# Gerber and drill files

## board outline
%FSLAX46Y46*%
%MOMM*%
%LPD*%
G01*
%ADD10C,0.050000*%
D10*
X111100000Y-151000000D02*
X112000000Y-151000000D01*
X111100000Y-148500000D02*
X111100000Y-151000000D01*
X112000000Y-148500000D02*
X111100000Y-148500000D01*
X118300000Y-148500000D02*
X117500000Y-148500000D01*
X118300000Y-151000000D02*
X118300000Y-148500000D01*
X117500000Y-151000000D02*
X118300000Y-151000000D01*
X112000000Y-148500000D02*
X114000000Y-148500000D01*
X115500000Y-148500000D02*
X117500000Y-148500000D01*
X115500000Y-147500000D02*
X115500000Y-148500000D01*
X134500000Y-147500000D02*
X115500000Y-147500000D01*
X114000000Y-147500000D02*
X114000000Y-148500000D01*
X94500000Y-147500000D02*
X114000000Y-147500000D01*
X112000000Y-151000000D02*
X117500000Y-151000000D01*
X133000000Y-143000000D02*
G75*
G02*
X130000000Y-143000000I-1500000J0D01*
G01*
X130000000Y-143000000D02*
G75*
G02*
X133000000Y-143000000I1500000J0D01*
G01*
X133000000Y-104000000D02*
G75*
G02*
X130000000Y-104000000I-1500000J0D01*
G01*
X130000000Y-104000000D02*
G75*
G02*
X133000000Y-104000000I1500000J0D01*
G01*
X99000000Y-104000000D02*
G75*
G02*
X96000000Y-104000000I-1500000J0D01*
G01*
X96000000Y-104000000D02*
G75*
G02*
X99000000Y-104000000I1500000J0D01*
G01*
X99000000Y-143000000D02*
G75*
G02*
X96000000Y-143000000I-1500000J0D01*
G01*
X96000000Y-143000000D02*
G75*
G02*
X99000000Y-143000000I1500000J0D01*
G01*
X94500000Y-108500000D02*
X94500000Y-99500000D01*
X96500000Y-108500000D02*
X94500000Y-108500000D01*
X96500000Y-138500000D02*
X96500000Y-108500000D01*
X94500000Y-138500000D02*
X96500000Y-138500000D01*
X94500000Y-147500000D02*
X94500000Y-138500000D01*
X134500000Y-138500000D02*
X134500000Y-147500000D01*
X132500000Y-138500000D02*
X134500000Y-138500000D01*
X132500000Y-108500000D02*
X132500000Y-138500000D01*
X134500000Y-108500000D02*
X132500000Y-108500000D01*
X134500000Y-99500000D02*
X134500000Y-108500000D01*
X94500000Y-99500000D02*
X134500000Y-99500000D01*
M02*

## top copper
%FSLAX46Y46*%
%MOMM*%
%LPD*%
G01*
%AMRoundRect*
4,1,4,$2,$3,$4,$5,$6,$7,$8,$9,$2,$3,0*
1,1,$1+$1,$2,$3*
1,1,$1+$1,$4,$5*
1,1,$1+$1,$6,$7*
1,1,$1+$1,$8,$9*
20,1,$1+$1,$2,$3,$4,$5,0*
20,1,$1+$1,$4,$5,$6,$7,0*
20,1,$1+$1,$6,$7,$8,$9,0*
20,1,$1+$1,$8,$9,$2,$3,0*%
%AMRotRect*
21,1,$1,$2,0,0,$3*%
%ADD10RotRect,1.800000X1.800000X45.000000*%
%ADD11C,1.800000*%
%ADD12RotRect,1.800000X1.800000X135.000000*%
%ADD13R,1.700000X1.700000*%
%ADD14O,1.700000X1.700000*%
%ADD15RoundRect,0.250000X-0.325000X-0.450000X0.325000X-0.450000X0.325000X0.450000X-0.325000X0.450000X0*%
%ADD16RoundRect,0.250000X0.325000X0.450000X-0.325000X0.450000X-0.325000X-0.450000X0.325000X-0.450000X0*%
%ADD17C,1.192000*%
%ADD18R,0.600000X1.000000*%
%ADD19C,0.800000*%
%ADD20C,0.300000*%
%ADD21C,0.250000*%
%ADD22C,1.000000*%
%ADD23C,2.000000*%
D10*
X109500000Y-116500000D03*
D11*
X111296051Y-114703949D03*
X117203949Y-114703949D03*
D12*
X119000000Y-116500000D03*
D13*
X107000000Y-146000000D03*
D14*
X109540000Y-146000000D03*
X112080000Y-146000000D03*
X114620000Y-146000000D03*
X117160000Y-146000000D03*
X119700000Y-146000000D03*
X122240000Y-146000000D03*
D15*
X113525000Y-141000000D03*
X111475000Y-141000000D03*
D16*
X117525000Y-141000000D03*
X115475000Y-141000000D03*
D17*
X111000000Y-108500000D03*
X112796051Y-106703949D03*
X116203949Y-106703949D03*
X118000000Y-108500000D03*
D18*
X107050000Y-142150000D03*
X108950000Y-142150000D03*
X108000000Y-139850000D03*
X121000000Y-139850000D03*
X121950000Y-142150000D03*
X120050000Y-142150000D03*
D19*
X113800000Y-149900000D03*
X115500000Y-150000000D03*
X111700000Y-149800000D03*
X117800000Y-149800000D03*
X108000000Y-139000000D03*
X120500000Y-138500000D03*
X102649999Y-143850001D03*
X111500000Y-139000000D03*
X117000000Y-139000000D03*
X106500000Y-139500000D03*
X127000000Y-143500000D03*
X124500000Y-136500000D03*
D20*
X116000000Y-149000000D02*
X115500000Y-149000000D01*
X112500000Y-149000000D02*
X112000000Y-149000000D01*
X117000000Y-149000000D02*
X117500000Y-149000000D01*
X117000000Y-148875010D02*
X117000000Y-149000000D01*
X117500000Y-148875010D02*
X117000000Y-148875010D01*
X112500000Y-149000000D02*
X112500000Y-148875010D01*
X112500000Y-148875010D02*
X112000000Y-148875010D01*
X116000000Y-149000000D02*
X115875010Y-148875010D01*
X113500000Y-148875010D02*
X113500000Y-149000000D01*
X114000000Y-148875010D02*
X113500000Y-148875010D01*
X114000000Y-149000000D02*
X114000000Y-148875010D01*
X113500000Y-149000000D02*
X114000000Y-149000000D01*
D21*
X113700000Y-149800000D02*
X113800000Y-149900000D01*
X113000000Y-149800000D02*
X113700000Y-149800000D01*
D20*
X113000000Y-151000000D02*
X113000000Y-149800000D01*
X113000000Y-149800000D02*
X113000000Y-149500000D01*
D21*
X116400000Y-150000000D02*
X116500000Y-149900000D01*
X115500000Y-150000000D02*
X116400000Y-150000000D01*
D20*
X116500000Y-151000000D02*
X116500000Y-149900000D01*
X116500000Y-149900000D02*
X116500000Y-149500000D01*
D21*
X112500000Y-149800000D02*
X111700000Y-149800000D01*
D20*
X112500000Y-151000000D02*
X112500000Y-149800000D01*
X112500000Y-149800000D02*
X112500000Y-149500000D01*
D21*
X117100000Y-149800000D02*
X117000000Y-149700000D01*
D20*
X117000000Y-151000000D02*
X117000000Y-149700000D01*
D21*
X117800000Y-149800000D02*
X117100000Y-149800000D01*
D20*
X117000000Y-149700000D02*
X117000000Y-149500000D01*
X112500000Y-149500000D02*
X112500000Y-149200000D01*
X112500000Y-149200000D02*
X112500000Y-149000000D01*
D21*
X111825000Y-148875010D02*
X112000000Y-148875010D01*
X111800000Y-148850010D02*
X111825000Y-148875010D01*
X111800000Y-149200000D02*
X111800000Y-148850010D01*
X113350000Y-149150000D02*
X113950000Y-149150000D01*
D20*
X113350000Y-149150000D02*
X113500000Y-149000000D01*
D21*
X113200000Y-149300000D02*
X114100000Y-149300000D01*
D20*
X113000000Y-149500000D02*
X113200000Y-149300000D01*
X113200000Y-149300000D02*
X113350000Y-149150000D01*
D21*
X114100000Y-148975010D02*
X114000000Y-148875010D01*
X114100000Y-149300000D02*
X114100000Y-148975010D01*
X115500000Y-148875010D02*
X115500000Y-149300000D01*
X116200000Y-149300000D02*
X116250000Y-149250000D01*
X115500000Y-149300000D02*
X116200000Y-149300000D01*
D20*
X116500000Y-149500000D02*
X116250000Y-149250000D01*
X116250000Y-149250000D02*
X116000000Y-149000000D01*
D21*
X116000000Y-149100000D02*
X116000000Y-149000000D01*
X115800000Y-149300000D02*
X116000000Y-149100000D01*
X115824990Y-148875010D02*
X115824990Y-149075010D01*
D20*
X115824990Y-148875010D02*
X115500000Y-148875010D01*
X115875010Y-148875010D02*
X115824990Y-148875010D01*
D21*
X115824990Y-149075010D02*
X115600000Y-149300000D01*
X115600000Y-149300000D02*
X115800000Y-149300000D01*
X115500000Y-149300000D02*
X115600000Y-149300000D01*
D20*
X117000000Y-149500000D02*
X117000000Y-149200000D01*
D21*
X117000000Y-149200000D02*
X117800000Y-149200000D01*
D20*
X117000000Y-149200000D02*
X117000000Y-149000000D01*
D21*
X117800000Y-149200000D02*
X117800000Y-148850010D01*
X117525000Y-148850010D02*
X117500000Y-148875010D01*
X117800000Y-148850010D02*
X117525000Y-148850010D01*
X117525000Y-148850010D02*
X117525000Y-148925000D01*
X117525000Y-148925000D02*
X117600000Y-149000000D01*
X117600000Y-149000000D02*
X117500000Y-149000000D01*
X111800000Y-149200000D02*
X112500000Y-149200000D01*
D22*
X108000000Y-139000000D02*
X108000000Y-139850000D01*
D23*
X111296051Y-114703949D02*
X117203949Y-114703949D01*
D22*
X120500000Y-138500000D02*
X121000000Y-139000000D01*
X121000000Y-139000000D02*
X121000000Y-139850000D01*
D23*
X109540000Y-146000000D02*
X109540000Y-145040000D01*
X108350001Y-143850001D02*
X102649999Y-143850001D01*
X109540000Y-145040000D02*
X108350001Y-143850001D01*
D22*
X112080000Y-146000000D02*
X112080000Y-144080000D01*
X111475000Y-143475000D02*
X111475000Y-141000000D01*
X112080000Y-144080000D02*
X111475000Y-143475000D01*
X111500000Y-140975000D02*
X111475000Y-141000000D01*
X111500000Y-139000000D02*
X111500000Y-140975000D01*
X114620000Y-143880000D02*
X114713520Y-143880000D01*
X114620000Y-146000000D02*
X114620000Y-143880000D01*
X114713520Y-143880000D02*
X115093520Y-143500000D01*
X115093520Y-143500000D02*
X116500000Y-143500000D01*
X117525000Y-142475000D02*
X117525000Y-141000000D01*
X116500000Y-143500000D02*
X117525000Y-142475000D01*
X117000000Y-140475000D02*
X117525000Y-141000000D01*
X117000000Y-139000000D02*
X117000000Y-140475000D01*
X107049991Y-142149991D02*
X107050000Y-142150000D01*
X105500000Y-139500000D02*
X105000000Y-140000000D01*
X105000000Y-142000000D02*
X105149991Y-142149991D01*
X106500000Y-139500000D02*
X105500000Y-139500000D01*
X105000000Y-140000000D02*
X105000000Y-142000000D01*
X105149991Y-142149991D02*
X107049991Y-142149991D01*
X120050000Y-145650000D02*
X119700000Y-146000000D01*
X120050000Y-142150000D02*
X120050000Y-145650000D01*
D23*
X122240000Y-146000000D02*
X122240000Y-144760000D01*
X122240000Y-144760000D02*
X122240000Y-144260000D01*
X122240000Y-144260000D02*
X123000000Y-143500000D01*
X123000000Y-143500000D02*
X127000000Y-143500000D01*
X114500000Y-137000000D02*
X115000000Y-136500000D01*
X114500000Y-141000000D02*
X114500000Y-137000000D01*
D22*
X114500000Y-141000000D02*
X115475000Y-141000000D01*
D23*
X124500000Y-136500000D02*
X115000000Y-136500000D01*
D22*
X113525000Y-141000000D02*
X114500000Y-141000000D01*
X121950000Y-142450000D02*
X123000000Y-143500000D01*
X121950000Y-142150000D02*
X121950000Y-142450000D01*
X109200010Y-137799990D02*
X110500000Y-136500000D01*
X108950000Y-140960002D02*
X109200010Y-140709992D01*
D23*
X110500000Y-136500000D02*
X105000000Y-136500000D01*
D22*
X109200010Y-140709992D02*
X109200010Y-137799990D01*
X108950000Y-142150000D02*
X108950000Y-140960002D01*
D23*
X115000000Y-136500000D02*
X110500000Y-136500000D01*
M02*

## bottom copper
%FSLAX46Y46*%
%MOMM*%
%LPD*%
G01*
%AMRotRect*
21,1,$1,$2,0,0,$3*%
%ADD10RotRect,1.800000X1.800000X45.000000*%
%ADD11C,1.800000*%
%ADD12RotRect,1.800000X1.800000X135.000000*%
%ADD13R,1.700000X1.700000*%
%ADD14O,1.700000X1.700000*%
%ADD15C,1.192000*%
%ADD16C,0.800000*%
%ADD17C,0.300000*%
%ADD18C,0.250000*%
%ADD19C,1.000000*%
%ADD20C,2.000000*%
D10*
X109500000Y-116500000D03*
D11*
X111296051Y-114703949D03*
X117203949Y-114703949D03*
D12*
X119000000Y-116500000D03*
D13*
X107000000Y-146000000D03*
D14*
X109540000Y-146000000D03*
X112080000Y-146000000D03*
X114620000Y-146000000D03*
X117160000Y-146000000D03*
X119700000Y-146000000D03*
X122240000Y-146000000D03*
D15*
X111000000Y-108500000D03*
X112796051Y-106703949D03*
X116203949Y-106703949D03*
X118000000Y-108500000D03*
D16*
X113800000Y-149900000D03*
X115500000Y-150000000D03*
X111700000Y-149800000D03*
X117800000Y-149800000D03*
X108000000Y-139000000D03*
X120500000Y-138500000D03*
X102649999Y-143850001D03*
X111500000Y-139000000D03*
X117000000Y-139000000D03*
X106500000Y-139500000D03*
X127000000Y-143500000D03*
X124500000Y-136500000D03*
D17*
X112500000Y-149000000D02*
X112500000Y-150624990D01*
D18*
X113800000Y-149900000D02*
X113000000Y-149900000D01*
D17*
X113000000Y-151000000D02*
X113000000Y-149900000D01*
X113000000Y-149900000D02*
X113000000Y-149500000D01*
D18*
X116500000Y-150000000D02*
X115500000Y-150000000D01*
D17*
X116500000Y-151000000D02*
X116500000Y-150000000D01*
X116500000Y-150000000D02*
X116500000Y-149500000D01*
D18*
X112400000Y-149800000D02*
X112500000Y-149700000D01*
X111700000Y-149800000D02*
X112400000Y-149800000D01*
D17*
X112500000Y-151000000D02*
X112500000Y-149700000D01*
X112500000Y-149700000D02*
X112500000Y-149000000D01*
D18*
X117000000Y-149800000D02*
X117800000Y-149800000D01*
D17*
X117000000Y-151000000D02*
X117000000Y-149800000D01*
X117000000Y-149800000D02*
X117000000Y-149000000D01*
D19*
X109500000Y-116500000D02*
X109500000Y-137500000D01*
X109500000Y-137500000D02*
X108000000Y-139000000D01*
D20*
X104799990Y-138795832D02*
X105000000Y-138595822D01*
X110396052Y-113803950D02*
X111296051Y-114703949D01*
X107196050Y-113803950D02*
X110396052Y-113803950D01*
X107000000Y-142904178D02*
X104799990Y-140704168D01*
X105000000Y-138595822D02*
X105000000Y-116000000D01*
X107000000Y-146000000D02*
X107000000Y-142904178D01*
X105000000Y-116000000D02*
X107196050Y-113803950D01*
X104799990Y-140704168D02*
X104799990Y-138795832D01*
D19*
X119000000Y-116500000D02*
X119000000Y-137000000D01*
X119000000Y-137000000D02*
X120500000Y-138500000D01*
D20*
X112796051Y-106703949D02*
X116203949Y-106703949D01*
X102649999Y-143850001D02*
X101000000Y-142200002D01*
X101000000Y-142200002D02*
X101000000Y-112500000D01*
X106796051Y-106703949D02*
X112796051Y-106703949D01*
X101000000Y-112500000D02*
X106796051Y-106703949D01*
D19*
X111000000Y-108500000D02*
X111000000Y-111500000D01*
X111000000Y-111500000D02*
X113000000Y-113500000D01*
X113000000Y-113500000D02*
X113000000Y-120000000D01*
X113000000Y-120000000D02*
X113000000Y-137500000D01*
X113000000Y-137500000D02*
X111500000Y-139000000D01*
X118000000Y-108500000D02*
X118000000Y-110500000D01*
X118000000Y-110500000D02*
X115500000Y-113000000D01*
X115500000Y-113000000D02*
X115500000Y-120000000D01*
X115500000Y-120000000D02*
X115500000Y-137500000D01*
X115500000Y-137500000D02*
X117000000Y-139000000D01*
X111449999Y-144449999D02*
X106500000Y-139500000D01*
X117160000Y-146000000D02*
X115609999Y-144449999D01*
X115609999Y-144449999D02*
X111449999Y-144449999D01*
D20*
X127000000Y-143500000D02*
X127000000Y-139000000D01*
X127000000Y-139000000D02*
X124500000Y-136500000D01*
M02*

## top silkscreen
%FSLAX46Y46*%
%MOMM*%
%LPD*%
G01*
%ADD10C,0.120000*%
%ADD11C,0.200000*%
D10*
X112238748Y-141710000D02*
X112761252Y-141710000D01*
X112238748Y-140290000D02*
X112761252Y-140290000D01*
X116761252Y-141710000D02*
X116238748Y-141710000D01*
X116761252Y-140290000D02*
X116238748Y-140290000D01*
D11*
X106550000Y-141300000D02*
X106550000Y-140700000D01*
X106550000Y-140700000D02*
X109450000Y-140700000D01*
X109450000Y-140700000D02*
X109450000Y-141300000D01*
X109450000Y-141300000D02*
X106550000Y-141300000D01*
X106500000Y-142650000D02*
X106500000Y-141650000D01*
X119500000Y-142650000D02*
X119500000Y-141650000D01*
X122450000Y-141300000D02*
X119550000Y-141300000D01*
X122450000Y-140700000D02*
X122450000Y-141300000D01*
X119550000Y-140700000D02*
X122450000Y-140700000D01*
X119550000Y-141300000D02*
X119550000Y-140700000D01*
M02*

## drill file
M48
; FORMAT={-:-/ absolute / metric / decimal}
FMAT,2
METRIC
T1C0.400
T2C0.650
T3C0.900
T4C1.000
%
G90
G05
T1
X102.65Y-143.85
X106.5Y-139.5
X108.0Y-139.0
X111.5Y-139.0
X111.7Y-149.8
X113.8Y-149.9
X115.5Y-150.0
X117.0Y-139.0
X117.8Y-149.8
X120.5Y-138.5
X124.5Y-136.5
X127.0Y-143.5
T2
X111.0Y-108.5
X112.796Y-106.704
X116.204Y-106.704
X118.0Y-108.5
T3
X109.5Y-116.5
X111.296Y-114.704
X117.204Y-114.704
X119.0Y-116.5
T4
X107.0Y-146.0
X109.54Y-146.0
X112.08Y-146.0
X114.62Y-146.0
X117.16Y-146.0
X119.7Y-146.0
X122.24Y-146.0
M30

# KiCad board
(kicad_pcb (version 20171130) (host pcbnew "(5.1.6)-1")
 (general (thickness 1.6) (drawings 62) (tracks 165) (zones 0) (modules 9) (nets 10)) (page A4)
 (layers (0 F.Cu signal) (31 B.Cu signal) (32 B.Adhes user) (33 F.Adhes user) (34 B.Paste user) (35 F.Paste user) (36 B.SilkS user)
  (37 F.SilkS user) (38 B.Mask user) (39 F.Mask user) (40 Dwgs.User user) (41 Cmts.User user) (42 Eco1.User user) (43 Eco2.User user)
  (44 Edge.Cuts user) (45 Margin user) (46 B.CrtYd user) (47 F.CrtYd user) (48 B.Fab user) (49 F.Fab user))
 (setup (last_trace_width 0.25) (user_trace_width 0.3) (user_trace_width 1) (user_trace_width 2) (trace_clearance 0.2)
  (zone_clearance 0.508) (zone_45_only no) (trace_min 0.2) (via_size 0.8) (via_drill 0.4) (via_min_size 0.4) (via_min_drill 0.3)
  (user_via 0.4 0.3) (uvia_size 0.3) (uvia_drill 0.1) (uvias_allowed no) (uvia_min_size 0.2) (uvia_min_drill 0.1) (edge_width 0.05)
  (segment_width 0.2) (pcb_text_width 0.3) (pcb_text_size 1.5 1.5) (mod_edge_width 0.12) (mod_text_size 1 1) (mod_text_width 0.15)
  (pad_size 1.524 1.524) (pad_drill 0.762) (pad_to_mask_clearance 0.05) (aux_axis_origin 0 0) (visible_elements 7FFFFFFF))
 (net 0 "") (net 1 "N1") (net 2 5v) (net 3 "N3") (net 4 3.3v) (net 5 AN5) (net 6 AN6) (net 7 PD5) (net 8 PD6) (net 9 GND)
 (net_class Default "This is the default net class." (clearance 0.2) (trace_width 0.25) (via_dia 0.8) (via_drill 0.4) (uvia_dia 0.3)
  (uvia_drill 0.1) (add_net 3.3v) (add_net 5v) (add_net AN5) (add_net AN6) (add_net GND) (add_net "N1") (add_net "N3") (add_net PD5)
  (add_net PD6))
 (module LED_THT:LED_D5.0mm (layer B.Cu) (at 109.5 116.5 45)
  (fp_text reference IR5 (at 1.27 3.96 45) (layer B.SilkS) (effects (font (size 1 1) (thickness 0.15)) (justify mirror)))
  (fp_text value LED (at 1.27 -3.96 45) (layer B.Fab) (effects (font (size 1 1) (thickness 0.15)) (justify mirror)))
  (pad 1 thru_hole rect (at 0 0 45) (size 1.8 1.8) (drill 0.9) (layers *.Cu *.Mask) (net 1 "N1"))
  (pad 2 thru_hole circle (at 2.54 0 45) (size 1.8 1.8) (drill 0.9) (layers *.Cu *.Mask) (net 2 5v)))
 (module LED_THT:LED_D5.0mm (layer B.Cu) (at 119 116.5 135)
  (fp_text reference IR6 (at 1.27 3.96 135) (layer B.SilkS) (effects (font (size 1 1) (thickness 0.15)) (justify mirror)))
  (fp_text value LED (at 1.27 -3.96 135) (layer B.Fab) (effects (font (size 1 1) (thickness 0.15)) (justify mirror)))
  (pad 2 thru_hole circle (at 2.54 0 135) (size 1.8 1.8) (drill 0.9) (layers *.Cu *.Mask) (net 2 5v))
  (pad 1 thru_hole rect (at 0 0 135) (size 1.8 1.8) (drill 0.9) (layers *.Cu *.Mask) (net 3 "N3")))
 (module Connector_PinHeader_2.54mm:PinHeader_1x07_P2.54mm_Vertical (layer B.Cu) (at 107 146 270)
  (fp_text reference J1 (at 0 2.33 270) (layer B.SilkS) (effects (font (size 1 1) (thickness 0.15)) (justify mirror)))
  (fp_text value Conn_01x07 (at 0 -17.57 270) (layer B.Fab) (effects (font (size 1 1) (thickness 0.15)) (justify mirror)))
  (pad 1 thru_hole rect (at 0 0 270) (size 1.7 1.7) (drill 1) (layers *.Cu *.Mask) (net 2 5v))
  (pad 2 thru_hole oval (at 0 -2.54 270) (size 1.7 1.7) (drill 1) (layers *.Cu *.Mask) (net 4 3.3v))
  (pad 3 thru_hole oval (at 0 -5.08 270) (size 1.7 1.7) (drill 1) (layers *.Cu *.Mask) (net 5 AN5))
  (pad 4 thru_hole oval (at 0 -7.62 270) (size 1.7 1.7) (drill 1) (layers *.Cu *.Mask) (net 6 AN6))
  (pad 5 thru_hole oval (at 0 -10.16 270) (size 1.7 1.7) (drill 1) (layers *.Cu *.Mask) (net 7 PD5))
  (pad 6 thru_hole oval (at 0 -12.7 270) (size 1.7 1.7) (drill 1) (layers *.Cu *.Mask) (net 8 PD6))
  (pad 7 thru_hole oval (at 0 -15.24 270) (size 1.7 1.7) (drill 1) (layers *.Cu *.Mask) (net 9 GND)))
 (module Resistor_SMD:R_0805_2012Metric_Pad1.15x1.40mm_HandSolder (layer F.Cu) (at 112.5 141)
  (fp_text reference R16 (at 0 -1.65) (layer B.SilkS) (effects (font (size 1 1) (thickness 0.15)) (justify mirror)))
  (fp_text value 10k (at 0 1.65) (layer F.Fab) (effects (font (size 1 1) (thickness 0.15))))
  (fp_line (start -0.261252 0.71) (end 0.261252 0.71) (layer F.SilkS) (width 0.12))
  (fp_line (start -0.261252 -0.71) (end 0.261252 -0.71) (layer F.SilkS) (width 0.12))
  (pad 2 smd roundrect (at 1.025 0) (size 1.15 1.4) (layers F.Cu F.Paste F.Mask) (roundrect_rratio 0.217391) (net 9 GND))
  (pad 1 smd roundrect (at -1.025 0) (size 1.15 1.4) (layers F.Cu F.Paste F.Mask) (roundrect_rratio 0.217391) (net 5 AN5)))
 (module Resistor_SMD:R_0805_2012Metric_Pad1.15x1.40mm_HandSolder (layer F.Cu) (at 116.5 141 180)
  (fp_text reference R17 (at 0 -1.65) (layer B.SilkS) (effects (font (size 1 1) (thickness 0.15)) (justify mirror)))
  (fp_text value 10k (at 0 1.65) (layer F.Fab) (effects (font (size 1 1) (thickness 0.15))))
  (fp_line (start -0.261252 -0.71) (end 0.261252 -0.71) (layer F.SilkS) (width 0.12))
  (fp_line (start -0.261252 0.71) (end 0.261252 0.71) (layer F.SilkS) (width 0.12))
  (pad 1 smd roundrect (at -1.025 0 180) (size 1.15 1.4) (layers F.Cu F.Paste F.Mask) (roundrect_rratio 0.217391) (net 6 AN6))
  (pad 2 smd roundrect (at 1.025 0 180) (size 1.15 1.4) (layers F.Cu F.Paste F.Mask) (roundrect_rratio 0.217391) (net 9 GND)))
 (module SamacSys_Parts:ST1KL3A (layer B.Cu) (at 111 108.5 45)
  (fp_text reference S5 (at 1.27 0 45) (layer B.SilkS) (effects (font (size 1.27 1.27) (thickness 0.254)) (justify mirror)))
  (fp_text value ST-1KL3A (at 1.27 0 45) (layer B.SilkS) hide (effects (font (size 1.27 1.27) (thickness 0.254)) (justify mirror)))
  (pad 1 thru_hole circle (at 0 0 45) (size 1.192 1.192) (drill 0.65) (layers *.Cu *.Mask) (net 5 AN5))
  (pad 2 thru_hole circle (at 2.54 0 45) (size 1.192 1.192) (drill 0.65) (layers *.Cu *.Mask) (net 4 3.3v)))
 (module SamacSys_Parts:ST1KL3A (layer B.Cu) (at 118 108.5 135)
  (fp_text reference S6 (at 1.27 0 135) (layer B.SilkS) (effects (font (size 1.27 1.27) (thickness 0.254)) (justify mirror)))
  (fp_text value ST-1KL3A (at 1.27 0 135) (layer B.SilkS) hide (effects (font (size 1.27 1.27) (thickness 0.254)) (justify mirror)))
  (pad 2 thru_hole circle (at 2.54 0 135) (size 1.192 1.192) (drill 0.65) (layers *.Cu *.Mask) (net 4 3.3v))
  (pad 1 thru_hole circle (at 0 0 135) (size 1.192 1.192) (drill 0.65) (layers *.Cu *.Mask) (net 6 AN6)))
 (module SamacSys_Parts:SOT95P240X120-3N (layer F.Cu) (at 108 141 90)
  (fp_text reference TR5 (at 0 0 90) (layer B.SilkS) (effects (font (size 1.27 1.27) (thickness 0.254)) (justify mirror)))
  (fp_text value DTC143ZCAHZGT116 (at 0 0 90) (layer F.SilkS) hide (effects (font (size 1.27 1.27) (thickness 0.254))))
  (fp_line (start -0.3 -1.45) (end 0.3 -1.45) (layer F.SilkS) (width 0.2))
  (fp_line (start 0.3 -1.45) (end 0.3 1.45) (layer F.SilkS) (width 0.2))
  (fp_line (start 0.3 1.45) (end -0.3 1.45) (layer F.SilkS) (width 0.2))
  (fp_line (start -0.3 1.45) (end -0.3 -1.45) (layer F.SilkS) (width 0.2))
  (fp_line (start -1.65 -1.5) (end -0.65 -1.5) (layer F.SilkS) (width 0.2))
  (pad 1 smd rect (at -1.15 -0.95 180) (size 0.6 1) (layers F.Cu F.Paste F.Mask) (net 7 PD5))
  (pad 2 smd rect (at -1.15 0.95 180) (size 0.6 1) (layers F.Cu F.Paste F.Mask) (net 9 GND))
  (pad 3 smd rect (at 1.15 0 180) (size 0.6 1) (layers F.Cu F.Paste F.Mask) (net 1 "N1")))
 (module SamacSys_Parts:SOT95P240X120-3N (layer F.Cu) (at 121 141 90)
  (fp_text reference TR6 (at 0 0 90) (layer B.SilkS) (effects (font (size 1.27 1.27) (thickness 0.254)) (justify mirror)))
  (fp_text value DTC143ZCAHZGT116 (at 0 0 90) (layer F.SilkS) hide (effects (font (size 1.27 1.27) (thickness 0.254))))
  (fp_line (start -1.65 -1.5) (end -0.65 -1.5) (layer F.SilkS) (width 0.2))
  (fp_line (start -0.3 1.45) (end -0.3 -1.45) (layer F.SilkS) (width 0.2))
  (fp_line (start 0.3 1.45) (end -0.3 1.45) (layer F.SilkS) (width 0.2))
  (fp_line (start 0.3 -1.45) (end 0.3 1.45) (layer F.SilkS) (width 0.2))
  (fp_line (start -0.3 -1.45) (end 0.3 -1.45) (layer F.SilkS) (width 0.2))
  (pad 3 smd rect (at 1.15 0 180) (size 0.6 1) (layers F.Cu F.Paste F.Mask) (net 3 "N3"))
  (pad 2 smd rect (at -1.15 0.95 180) (size 0.6 1) (layers F.Cu F.Paste F.Mask) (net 9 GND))
  (pad 1 smd rect (at -1.15 -0.95 180) (size 0.6 1) (layers F.Cu F.Paste F.Mask) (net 8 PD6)))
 (gr_line (start 111.1 151) (end 112 151) (layer Edge.Cuts) (width 0.05))
 (gr_line (start 111.1 148.5) (end 111.1 151) (layer Edge.Cuts) (width 0.05))
 (gr_line (start 112 148.5) (end 111.1 148.5) (layer Edge.Cuts) (width 0.05))
 (gr_line (start 118.3 148.5) (end 117.5 148.5) (layer Edge.Cuts) (width 0.05))
 (gr_line (start 118.3 151) (end 118.3 148.5) (layer Edge.Cuts) (width 0.05))
 (gr_line (start 117.5 151) (end 118.3 151) (layer Edge.Cuts) (width 0.05))
 (gr_line (start 112 148.5) (end 114 148.5) (layer Edge.Cuts) (width 0.05))
 (gr_line (start 115.5 148.5) (end 117.5 148.5) (layer Edge.Cuts) (width 0.05))
 (gr_line (start 115.5 147.5) (end 115.5 148.5) (layer Edge.Cuts) (width 0.05))
 (gr_line (start 134.5 147.5) (end 115.5 147.5) (layer Edge.Cuts) (width 0.05))
 (gr_line (start 114 147.5) (end 114 148.5) (layer Edge.Cuts) (width 0.05))
 (gr_line (start 94.5 147.5) (end 114 147.5) (layer Edge.Cuts) (width 0.05))
 (gr_line (start 112 151) (end 117.5 151) (layer Edge.Cuts) (width 0.05))
 (gr_circle (center 131.5 143) (end 130 143) (layer Edge.Cuts) (width 0.05))
 (gr_circle (center 131.5 104) (end 130 104) (layer Edge.Cuts) (width 0.05))
 (gr_circle (center 97.5 104) (end 99 104) (layer Edge.Cuts) (width 0.05))
 (gr_circle (center 97.5 143) (end 99 143) (layer Edge.Cuts) (width 0.05))
 (gr_line (start 94.5 108.5) (end 94.5 99.5) (layer Edge.Cuts) (width 0.05))
 (gr_line (start 96.5 108.5) (end 94.5 108.5) (layer Edge.Cuts) (width 0.05))
 (gr_line (start 96.5 138.5) (end 96.5 108.5) (layer Edge.Cuts) (width 0.05))
 (gr_line (start 94.5 138.5) (end 96.5 138.5) (layer Edge.Cuts) (width 0.05))
 (gr_line (start 94.5 147.5) (end 94.5 138.5) (layer Edge.Cuts) (width 0.05))
 (gr_line (start 134.5 138.5) (end 134.5 147.5) (layer Edge.Cuts) (width 0.05))
 (gr_line (start 132.5 138.5) (end 134.5 138.5) (layer Edge.Cuts) (width 0.05))
 (gr_line (start 132.5 108.5) (end 132.5 138.5) (layer Edge.Cuts) (width 0.05))
 (gr_line (start 134.5 108.5) (end 132.5 108.5) (layer Edge.Cuts) (width 0.05))
 (gr_line (start 134.5 99.5) (end 134.5 108.5) (layer Edge.Cuts) (width 0.05))
 (gr_line (start 94.5 99.5) (end 134.5 99.5) (layer Edge.Cuts) (width 0.05))
 (segment (start 116 149) (end 115.5 149) (width 0.3) (layer F.Cu) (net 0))
 (segment (start 112.5 149) (end 112.5 150.62499) (width 0.3) (layer B.Cu) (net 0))
 (segment (start 112.5 149) (end 112 149) (width 0.3) (layer F.Cu) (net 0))
 (segment (start 117 149) (end 117.5 149) (width 0.3) (layer F.Cu) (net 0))
 (segment (start 117 148.87501) (end 117 149) (width 0.3) (layer F.Cu) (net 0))
 (segment (start 117.5 148.87501) (end 117 148.87501) (width 0.3) (layer F.Cu) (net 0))
 (segment (start 112.5 149) (end 112.5 148.87501) (width 0.3) (layer F.Cu) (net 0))
 (segment (start 112.5 148.87501) (end 112 148.87501) (width 0.3) (layer F.Cu) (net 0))
 (segment (start 116 149) (end 115.87501 148.87501) (width 0.3) (layer F.Cu) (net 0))
 (segment (start 113.5 148.87501) (end 113.5 149) (width 0.3) (layer F.Cu) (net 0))
 (segment (start 114 148.87501) (end 113.5 148.87501) (width 0.3) (layer F.Cu) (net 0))
 (segment (start 114 149) (end 114 148.87501) (width 0.3) (layer F.Cu) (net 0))
 (segment (start 113.5 149) (end 114 149) (width 0.3) (layer F.Cu) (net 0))
 (via (at 113.8 149.9) (size 0.8) (drill 0.4) (layers F.Cu B.Cu) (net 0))
 (segment (start 113.7 149.8) (end 113.8 149.9) (width 0.25) (layer F.Cu) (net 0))
 (segment (start 113 149.8) (end 113.7 149.8) (width 0.25) (layer F.Cu) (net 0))
 (segment (start 113 151) (end 113 149.8) (width 0.3) (layer F.Cu) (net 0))
 (segment (start 113 149.8) (end 113 149.5) (width 0.3) (layer F.Cu) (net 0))
 (segment (start 113.8 149.9) (end 113 149.9) (width 0.25) (layer B.Cu) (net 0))
 (segment (start 113 151) (end 113 149.9) (width 0.3) (layer B.Cu) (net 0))
 (segment (start 113 149.9) (end 113 149.5) (width 0.3) (layer B.Cu) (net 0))
 (via (at 115.5 150) (size 0.8) (drill 0.4) (layers F.Cu B.Cu) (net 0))
 (segment (start 116.5 150) (end 115.5 150) (width 0.25) (layer B.Cu) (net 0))
 (segment (start 116.5 151) (end 116.5 150) (width 0.3) (layer B.Cu) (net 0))
 (segment (start 116.5 150) (end 116.5 149.5) (width 0.3) (layer B.Cu) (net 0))
 (segment (start 116.4 150) (end 116.5 149.9) (width 0.25) (layer F.Cu) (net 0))
 (segment (start 115.5 150) (end 116.4 150) (width 0.25) (layer F.Cu) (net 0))
 (segment (start 116.5 151) (end 116.5 149.9) (width 0.3) (layer F.Cu) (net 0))
 (segment (start 116.5 149.9) (end 116.5 149.5) (width 0.3) (layer F.Cu) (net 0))
 (segment (start 112.5 149.8) (end 111.7 149.8) (width 0.25) (layer F.Cu) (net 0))
 (segment (start 112.5 151) (end 112.5 149.8) (width 0.3) (layer F.Cu) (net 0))
 (via (at 111.7 149.8) (size 0.8) (drill 0.4) (layers F.Cu B.Cu) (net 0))
 (segment (start 112.5 149.8) (end 112.5 149.5) (width 0.3) (layer F.Cu) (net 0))
 (segment (start 112.4 149.8) (end 112.5 149.7) (width 0.25) (layer B.Cu) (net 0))
 (segment (start 111.7 149.8) (end 112.4 149.8) (width 0.25) (layer B.Cu) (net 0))
 (segment (start 112.5 151) (end 112.5 149.7) (width 0.3) (layer B.Cu) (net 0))
 (segment (start 112.5 149.7) (end 112.5 149) (width 0.3) (layer B.Cu) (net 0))
 (via (at 117.8 149.8) (size 0.8) (drill 0.4) (layers F.Cu B.Cu) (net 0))
 (segment (start 117 149.8) (end 117.8 149.8) (width 0.25) (layer B.Cu) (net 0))
 (segment (start 117 151) (end 117 149.8) (width 0.3) (layer B.Cu) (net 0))
 (segment (start 117 149.8) (end 117 149) (width 0.3) (layer B.Cu) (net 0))
 (segment (start 117.1 149.8) (end 117 149.7) (width 0.25) (layer F.Cu) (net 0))
 (segment (start 117 151) (end 117 149.7) (width 0.3) (layer F.Cu) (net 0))
 (segment (start 117.8 149.8) (end 117.1 149.8) (width 0.25) (layer F.Cu) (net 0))
 (segment (start 117 149.7) (end 117 149.5) (width 0.3) (layer F.Cu) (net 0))
 (segment (start 112.5 149.5) (end 112.5 149.2) (width 0.3) (layer F.Cu) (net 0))
 (segment (start 112.5 149.2) (end 112.5 149) (width 0.3) (layer F.Cu) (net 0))
 (segment (start 111.825 148.87501) (end 112 148.87501) (width 0.25) (layer F.Cu) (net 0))
 (segment (start 111.8 148.85001) (end 111.825 148.87501) (width 0.25) (layer F.Cu) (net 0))
 (segment (start 111.8 149.2) (end 111.8 148.85001) (width 0.25) (layer F.Cu) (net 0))
 (segment (start 113.35 149.15) (end 113.95 149.15) (width 0.25) (layer F.Cu) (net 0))
 (segment (start 113.35 149.15) (end 113.5 149) (width 0.3) (layer F.Cu) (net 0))
 (segment (start 113.2 149.3) (end 114.1 149.3) (width 0.25) (layer F.Cu) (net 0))
 (segment (start 113 149.5) (end 113.2 149.3) (width 0.3) (layer F.Cu) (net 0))
 (segment (start 113.2 149.3) (end 113.35 149.15) (width 0.3) (layer F.Cu) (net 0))
 (segment (start 114.1 148.97501) (end 114 148.87501) (width 0.25) (layer F.Cu) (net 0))
 (segment (start 114.1 149.3) (end 114.1 148.97501) (width 0.25) (layer F.Cu) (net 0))
 (segment (start 115.5 148.87501) (end 115.5 149.3) (width 0.25) (layer F.Cu) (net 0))
 (segment (start 116.2 149.3) (end 116.25 149.25) (width 0.25) (layer F.Cu) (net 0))
 (segment (start 115.5 149.3) (end 116.2 149.3) (width 0.25) (layer F.Cu) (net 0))
 (segment (start 116.5 149.5) (end 116.25 149.25) (width 0.3) (layer F.Cu) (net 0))
 (segment (start 116.25 149.25) (end 116 149) (width 0.3) (layer F.Cu) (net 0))
 (segment (start 116 149.1) (end 116 149) (width 0.25) (layer F.Cu) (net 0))
 (segment (start 115.8 149.3) (end 116 149.1) (width 0.25) (layer F.Cu) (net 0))
 (segment (start 115.82499 148.87501) (end 115.82499 149.07501) (width 0.25) (layer F.Cu) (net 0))
 (segment (start 115.82499 148.87501) (end 115.5 148.87501) (width 0.3) (layer F.Cu) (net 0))
 (segment (start 115.87501 148.87501) (end 115.82499 148.87501) (width 0.3) (layer F.Cu) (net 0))
 (segment (start 115.82499 149.07501) (end 115.6 149.3) (width 0.25) (layer F.Cu) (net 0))
 (segment (start 115.6 149.3) (end 115.8 149.3) (width 0.25) (layer F.Cu) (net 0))
 (segment (start 115.5 149.3) (end 115.6 149.3) (width 0.25) (layer F.Cu) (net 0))
 (segment (start 117 149.5) (end 117 149.2) (width 0.3) (layer F.Cu) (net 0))
 (segment (start 117 149.2) (end 117.8 149.2) (width 0.25) (layer F.Cu) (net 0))
 (segment (start 117 149.2) (end 117 149) (width 0.3) (layer F.Cu) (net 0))
 (segment (start 117.8 149.2) (end 117.8 148.85001) (width 0.25) (layer F.Cu) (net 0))
 (segment (start 117.525 148.85001) (end 117.5 148.87501) (width 0.25) (layer F.Cu) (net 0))
 (segment (start 117.8 148.85001) (end 117.525 148.85001) (width 0.25) (layer F.Cu) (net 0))
 (segment (start 117.525 148.85001) (end 117.525 148.925) (width 0.25) (layer F.Cu) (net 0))
 (segment (start 117.525 148.925) (end 117.6 149) (width 0.25) (layer F.Cu) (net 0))
 (segment (start 117.6 149) (end 117.5 149) (width 0.25) (layer F.Cu) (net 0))
 (segment (start 111.8 149.2) (end 112.5 149.2) (width 0.25) (layer F.Cu) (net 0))
 (segment (start 109.5 116.5) (end 109.5 137.5) (width 1) (layer B.Cu) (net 1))
 (via (at 108 139) (size 0.8) (drill 0.4) (layers F.Cu B.Cu) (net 1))
 (segment (start 109.5 137.5) (end 108 139) (width 1) (layer B.Cu) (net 1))
 (segment (start 108 139) (end 108 139.85) (width 1) (layer F.Cu) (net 1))
 (segment (start 111.296051 114.703949) (end 117.203949 114.703949) (width 2) (layer F.Cu) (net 2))
 (segment (start 104.79999 138.795832) (end 105 138.595822) (width 2) (layer B.Cu) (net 2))
 (segment (start 110.396052 113.80395) (end 111.296051 114.703949) (width 2) (layer B.Cu) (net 2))
 (segment (start 107.19605 113.80395) (end 110.396052 113.80395) (width 2) (layer B.Cu) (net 2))
 (segment (start 107 142.904178) (end 104.79999 140.704168) (width 2) (layer B.Cu) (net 2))
 (segment (start 105 138.595822) (end 105 116) (width 2) (layer B.Cu) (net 2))
 (segment (start 107 146) (end 107 142.904178) (width 2) (layer B.Cu) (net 2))
 (segment (start 105 116) (end 107.19605 113.80395) (width 2) (layer B.Cu) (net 2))
 (segment (start 104.79999 140.704168) (end 104.79999 138.795832) (width 2) (layer B.Cu) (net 2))
 (segment (start 119 116.5) (end 119 137) (width 1) (layer B.Cu) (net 3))
 (via (at 120.5 138.5) (size 0.8) (drill 0.4) (layers F.Cu B.Cu) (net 3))
 (segment (start 119 137) (end 120.5 138.5) (width 1) (layer B.Cu) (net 3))
 (segment (start 120.5 138.5) (end 121 139) (width 1) (layer F.Cu) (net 3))
 (segment (start 121 139) (end 121 139.85) (width 1) (layer F.Cu) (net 3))
 (segment (start 112.796051 106.703949) (end 116.203949 106.703949) (width 2) (layer B.Cu) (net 4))
 (segment (start 109.54 146) (end 109.54 145.04) (width 2) (layer F.Cu) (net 4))
 (segment (start 108.350001 143.850001) (end 102.649999 143.850001) (width 2) (layer F.Cu) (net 4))
 (segment (start 109.54 145.04) (end 108.350001 143.850001) (width 2) (layer F.Cu) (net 4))
 (via (at 102.649999 143.850001) (size 0.8) (drill 0.4) (layers F.Cu B.Cu) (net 4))
 (segment (start 102.649999 143.850001) (end 101 142.200002) (width 2) (layer B.Cu) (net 4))
 (segment (start 101 142.200002) (end 101 112.5) (width 2) (layer B.Cu) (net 4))
 (segment (start 106.796051 106.703949) (end 112.796051 106.703949) (width 2) (layer B.Cu) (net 4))
 (segment (start 101 112.5) (end 106.796051 106.703949) (width 2) (layer B.Cu) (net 4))
 (segment (start 112.08 146) (end 112.08 144.08) (width 1) (layer F.Cu) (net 5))
 (segment (start 111.475 143.475) (end 111.475 141) (width 1) (layer F.Cu) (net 5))
 (segment (start 112.08 144.08) (end 111.475 143.475) (width 1) (layer F.Cu) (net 5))
 (segment (start 111 108.5) (end 111 111.5) (width 1) (layer B.Cu) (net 5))
 (segment (start 111 111.5) (end 113 113.5) (width 1) (layer B.Cu) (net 5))
 (segment (start 113 113.5) (end 113 120) (width 1) (layer B.Cu) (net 5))
 (segment (start 113 120) (end 113 137.5) (width 1) (layer B.Cu) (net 5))
 (via (at 111.5 139) (size 0.8) (drill 0.4) (layers F.Cu B.Cu) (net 5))
 (segment (start 113 137.5) (end 111.5 139) (width 1) (layer B.Cu) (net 5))
 (segment (start 111.5 140.975) (end 111.475 141) (width 1) (layer F.Cu) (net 5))
 (segment (start 111.5 139) (end 111.5 140.975) (width 1) (layer F.Cu) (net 5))
 (segment (start 114.62 143.88) (end 114.71352 143.88) (width 1) (layer F.Cu) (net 6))
 (segment (start 114.62 146) (end 114.62 143.88) (width 1) (layer F.Cu) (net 6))
 (segment (start 114.71352 143.88) (end 115.09352 143.5) (width 1) (layer F.Cu) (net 6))
 (segment (start 115.09352 143.5) (end 116.5 143.5) (width 1) (layer F.Cu) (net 6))
 (segment (start 117.525 142.475) (end 117.525 141) (width 1) (layer F.Cu) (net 6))
 (segment (start 116.5 143.5) (end 117.525 142.475) (width 1) (layer F.Cu) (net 6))
 (segment (start 118 108.5) (end 118 110.5) (width 1) (layer B.Cu) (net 6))
 (segment (start 118 110.5) (end 115.5 113) (width 1) (layer B.Cu) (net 6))
 (segment (start 115.5 113) (end 115.5 120) (width 1) (layer B.Cu) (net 6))
 (via (at 117 139) (size 0.8) (drill 0.4) (layers F.Cu B.Cu) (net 6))
 (segment (start 115.5 120) (end 115.5 137.5) (width 1) (layer B.Cu) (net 6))
 (segment (start 115.5 137.5) (end 117 139) (width 1) (layer B.Cu) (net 6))
 (segment (start 117 140.475) (end 117.525 141) (width 1) (layer F.Cu) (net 6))
 (segment (start 117 139) (end 117 140.475) (width 1) (layer F.Cu) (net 6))
 (via (at 106.5 139.5) (size 0.8) (drill 0.4) (layers F.Cu B.Cu) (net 7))
 (segment (start 111.449999 144.449999) (end 106.5 139.5) (width 1) (layer B.Cu) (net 7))
 (segment (start 117.16 146) (end 115.609999 144.449999) (width 1) (layer B.Cu) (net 7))
 (segment (start 115.609999 144.449999) (end 111.449999 144.449999) (width 1) (layer B.Cu) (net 7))
 (segment (start 107.049991 142.149991) (end 107.05 142.15) (width 1) (layer F.Cu) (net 7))
 (segment (start 105.5 139.5) (end 105 140) (width 1) (layer F.Cu) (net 7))
 (segment (start 105 142) (end 105.149991 142.149991) (width 1) (layer F.Cu) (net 7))
 (segment (start 106.5 139.5) (end 105.5 139.5) (width 1) (layer F.Cu) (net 7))
 (segment (start 105 140) (end 105 142) (width 1) (layer F.Cu) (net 7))
 (segment (start 105.149991 142.149991) (end 107.049991 142.149991) (width 1) (layer F.Cu) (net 7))
 (segment (start 120.05 145.65) (end 119.7 146) (width 1) (layer F.Cu) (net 8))
 (segment (start 120.05 142.15) (end 120.05 145.65) (width 1) (layer F.Cu) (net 8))
 (segment (start 122.24 146) (end 122.24 144.76) (width 2) (layer F.Cu) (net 9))
 (segment (start 122.24 144.76) (end 122.24 144.26) (width 2) (layer F.Cu) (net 9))
 (segment (start 122.24 144.26) (end 123 143.5) (width 2) (layer F.Cu) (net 9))
 (via (at 127 143.5) (size 0.8) (drill 0.4) (layers F.Cu B.Cu) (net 9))
 (segment (start 123 143.5) (end 127 143.5) (width 2) (layer F.Cu) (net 9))
 (segment (start 127 143.5) (end 127 139) (width 2) (layer B.Cu) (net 9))
 (segment (start 127 139) (end 124.5 136.5) (width 2) (layer B.Cu) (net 9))
 (via (at 124.5 136.5) (size 0.8) (drill 0.4) (layers F.Cu B.Cu) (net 9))
 (segment (start 114.5 137) (end 115 136.5) (width 2) (layer F.Cu) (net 9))
 (segment (start 114.5 141) (end 114.5 137) (width 2) (layer F.Cu) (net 9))
 (segment (start 114.5 141) (end 115.475 141) (width 1) (layer F.Cu) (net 9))
 (segment (start 124.5 136.5) (end 115 136.5) (width 2) (layer F.Cu) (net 9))
 (segment (start 113.525 141) (end 114.5 141) (width 1) (layer F.Cu) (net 9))
 (segment (start 121.95 142.45) (end 123 143.5) (width 1) (layer F.Cu) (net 9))
 (segment (start 121.95 142.15) (end 121.95 142.45) (width 1) (layer F.Cu) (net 9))
 (segment (start 109.20001 137.79999) (end 110.5 136.5) (width 1) (layer F.Cu) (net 9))
 (segment (start 108.95 140.960002) (end 109.20001 140.709992) (width 1) (layer F.Cu) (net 9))
 (segment (start 110.5 136.5) (end 105 136.5) (width 2) (layer F.Cu) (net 9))
 (segment (start 109.20001 140.709992) (end 109.20001 137.79999) (width 1) (layer F.Cu) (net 9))
 (segment (start 108.95 142.15) (end 108.95 140.960002) (width 1) (layer F.Cu) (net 9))
 (segment (start 115 136.5) (end 110.5 136.5) (width 2) (layer F.Cu) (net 9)))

